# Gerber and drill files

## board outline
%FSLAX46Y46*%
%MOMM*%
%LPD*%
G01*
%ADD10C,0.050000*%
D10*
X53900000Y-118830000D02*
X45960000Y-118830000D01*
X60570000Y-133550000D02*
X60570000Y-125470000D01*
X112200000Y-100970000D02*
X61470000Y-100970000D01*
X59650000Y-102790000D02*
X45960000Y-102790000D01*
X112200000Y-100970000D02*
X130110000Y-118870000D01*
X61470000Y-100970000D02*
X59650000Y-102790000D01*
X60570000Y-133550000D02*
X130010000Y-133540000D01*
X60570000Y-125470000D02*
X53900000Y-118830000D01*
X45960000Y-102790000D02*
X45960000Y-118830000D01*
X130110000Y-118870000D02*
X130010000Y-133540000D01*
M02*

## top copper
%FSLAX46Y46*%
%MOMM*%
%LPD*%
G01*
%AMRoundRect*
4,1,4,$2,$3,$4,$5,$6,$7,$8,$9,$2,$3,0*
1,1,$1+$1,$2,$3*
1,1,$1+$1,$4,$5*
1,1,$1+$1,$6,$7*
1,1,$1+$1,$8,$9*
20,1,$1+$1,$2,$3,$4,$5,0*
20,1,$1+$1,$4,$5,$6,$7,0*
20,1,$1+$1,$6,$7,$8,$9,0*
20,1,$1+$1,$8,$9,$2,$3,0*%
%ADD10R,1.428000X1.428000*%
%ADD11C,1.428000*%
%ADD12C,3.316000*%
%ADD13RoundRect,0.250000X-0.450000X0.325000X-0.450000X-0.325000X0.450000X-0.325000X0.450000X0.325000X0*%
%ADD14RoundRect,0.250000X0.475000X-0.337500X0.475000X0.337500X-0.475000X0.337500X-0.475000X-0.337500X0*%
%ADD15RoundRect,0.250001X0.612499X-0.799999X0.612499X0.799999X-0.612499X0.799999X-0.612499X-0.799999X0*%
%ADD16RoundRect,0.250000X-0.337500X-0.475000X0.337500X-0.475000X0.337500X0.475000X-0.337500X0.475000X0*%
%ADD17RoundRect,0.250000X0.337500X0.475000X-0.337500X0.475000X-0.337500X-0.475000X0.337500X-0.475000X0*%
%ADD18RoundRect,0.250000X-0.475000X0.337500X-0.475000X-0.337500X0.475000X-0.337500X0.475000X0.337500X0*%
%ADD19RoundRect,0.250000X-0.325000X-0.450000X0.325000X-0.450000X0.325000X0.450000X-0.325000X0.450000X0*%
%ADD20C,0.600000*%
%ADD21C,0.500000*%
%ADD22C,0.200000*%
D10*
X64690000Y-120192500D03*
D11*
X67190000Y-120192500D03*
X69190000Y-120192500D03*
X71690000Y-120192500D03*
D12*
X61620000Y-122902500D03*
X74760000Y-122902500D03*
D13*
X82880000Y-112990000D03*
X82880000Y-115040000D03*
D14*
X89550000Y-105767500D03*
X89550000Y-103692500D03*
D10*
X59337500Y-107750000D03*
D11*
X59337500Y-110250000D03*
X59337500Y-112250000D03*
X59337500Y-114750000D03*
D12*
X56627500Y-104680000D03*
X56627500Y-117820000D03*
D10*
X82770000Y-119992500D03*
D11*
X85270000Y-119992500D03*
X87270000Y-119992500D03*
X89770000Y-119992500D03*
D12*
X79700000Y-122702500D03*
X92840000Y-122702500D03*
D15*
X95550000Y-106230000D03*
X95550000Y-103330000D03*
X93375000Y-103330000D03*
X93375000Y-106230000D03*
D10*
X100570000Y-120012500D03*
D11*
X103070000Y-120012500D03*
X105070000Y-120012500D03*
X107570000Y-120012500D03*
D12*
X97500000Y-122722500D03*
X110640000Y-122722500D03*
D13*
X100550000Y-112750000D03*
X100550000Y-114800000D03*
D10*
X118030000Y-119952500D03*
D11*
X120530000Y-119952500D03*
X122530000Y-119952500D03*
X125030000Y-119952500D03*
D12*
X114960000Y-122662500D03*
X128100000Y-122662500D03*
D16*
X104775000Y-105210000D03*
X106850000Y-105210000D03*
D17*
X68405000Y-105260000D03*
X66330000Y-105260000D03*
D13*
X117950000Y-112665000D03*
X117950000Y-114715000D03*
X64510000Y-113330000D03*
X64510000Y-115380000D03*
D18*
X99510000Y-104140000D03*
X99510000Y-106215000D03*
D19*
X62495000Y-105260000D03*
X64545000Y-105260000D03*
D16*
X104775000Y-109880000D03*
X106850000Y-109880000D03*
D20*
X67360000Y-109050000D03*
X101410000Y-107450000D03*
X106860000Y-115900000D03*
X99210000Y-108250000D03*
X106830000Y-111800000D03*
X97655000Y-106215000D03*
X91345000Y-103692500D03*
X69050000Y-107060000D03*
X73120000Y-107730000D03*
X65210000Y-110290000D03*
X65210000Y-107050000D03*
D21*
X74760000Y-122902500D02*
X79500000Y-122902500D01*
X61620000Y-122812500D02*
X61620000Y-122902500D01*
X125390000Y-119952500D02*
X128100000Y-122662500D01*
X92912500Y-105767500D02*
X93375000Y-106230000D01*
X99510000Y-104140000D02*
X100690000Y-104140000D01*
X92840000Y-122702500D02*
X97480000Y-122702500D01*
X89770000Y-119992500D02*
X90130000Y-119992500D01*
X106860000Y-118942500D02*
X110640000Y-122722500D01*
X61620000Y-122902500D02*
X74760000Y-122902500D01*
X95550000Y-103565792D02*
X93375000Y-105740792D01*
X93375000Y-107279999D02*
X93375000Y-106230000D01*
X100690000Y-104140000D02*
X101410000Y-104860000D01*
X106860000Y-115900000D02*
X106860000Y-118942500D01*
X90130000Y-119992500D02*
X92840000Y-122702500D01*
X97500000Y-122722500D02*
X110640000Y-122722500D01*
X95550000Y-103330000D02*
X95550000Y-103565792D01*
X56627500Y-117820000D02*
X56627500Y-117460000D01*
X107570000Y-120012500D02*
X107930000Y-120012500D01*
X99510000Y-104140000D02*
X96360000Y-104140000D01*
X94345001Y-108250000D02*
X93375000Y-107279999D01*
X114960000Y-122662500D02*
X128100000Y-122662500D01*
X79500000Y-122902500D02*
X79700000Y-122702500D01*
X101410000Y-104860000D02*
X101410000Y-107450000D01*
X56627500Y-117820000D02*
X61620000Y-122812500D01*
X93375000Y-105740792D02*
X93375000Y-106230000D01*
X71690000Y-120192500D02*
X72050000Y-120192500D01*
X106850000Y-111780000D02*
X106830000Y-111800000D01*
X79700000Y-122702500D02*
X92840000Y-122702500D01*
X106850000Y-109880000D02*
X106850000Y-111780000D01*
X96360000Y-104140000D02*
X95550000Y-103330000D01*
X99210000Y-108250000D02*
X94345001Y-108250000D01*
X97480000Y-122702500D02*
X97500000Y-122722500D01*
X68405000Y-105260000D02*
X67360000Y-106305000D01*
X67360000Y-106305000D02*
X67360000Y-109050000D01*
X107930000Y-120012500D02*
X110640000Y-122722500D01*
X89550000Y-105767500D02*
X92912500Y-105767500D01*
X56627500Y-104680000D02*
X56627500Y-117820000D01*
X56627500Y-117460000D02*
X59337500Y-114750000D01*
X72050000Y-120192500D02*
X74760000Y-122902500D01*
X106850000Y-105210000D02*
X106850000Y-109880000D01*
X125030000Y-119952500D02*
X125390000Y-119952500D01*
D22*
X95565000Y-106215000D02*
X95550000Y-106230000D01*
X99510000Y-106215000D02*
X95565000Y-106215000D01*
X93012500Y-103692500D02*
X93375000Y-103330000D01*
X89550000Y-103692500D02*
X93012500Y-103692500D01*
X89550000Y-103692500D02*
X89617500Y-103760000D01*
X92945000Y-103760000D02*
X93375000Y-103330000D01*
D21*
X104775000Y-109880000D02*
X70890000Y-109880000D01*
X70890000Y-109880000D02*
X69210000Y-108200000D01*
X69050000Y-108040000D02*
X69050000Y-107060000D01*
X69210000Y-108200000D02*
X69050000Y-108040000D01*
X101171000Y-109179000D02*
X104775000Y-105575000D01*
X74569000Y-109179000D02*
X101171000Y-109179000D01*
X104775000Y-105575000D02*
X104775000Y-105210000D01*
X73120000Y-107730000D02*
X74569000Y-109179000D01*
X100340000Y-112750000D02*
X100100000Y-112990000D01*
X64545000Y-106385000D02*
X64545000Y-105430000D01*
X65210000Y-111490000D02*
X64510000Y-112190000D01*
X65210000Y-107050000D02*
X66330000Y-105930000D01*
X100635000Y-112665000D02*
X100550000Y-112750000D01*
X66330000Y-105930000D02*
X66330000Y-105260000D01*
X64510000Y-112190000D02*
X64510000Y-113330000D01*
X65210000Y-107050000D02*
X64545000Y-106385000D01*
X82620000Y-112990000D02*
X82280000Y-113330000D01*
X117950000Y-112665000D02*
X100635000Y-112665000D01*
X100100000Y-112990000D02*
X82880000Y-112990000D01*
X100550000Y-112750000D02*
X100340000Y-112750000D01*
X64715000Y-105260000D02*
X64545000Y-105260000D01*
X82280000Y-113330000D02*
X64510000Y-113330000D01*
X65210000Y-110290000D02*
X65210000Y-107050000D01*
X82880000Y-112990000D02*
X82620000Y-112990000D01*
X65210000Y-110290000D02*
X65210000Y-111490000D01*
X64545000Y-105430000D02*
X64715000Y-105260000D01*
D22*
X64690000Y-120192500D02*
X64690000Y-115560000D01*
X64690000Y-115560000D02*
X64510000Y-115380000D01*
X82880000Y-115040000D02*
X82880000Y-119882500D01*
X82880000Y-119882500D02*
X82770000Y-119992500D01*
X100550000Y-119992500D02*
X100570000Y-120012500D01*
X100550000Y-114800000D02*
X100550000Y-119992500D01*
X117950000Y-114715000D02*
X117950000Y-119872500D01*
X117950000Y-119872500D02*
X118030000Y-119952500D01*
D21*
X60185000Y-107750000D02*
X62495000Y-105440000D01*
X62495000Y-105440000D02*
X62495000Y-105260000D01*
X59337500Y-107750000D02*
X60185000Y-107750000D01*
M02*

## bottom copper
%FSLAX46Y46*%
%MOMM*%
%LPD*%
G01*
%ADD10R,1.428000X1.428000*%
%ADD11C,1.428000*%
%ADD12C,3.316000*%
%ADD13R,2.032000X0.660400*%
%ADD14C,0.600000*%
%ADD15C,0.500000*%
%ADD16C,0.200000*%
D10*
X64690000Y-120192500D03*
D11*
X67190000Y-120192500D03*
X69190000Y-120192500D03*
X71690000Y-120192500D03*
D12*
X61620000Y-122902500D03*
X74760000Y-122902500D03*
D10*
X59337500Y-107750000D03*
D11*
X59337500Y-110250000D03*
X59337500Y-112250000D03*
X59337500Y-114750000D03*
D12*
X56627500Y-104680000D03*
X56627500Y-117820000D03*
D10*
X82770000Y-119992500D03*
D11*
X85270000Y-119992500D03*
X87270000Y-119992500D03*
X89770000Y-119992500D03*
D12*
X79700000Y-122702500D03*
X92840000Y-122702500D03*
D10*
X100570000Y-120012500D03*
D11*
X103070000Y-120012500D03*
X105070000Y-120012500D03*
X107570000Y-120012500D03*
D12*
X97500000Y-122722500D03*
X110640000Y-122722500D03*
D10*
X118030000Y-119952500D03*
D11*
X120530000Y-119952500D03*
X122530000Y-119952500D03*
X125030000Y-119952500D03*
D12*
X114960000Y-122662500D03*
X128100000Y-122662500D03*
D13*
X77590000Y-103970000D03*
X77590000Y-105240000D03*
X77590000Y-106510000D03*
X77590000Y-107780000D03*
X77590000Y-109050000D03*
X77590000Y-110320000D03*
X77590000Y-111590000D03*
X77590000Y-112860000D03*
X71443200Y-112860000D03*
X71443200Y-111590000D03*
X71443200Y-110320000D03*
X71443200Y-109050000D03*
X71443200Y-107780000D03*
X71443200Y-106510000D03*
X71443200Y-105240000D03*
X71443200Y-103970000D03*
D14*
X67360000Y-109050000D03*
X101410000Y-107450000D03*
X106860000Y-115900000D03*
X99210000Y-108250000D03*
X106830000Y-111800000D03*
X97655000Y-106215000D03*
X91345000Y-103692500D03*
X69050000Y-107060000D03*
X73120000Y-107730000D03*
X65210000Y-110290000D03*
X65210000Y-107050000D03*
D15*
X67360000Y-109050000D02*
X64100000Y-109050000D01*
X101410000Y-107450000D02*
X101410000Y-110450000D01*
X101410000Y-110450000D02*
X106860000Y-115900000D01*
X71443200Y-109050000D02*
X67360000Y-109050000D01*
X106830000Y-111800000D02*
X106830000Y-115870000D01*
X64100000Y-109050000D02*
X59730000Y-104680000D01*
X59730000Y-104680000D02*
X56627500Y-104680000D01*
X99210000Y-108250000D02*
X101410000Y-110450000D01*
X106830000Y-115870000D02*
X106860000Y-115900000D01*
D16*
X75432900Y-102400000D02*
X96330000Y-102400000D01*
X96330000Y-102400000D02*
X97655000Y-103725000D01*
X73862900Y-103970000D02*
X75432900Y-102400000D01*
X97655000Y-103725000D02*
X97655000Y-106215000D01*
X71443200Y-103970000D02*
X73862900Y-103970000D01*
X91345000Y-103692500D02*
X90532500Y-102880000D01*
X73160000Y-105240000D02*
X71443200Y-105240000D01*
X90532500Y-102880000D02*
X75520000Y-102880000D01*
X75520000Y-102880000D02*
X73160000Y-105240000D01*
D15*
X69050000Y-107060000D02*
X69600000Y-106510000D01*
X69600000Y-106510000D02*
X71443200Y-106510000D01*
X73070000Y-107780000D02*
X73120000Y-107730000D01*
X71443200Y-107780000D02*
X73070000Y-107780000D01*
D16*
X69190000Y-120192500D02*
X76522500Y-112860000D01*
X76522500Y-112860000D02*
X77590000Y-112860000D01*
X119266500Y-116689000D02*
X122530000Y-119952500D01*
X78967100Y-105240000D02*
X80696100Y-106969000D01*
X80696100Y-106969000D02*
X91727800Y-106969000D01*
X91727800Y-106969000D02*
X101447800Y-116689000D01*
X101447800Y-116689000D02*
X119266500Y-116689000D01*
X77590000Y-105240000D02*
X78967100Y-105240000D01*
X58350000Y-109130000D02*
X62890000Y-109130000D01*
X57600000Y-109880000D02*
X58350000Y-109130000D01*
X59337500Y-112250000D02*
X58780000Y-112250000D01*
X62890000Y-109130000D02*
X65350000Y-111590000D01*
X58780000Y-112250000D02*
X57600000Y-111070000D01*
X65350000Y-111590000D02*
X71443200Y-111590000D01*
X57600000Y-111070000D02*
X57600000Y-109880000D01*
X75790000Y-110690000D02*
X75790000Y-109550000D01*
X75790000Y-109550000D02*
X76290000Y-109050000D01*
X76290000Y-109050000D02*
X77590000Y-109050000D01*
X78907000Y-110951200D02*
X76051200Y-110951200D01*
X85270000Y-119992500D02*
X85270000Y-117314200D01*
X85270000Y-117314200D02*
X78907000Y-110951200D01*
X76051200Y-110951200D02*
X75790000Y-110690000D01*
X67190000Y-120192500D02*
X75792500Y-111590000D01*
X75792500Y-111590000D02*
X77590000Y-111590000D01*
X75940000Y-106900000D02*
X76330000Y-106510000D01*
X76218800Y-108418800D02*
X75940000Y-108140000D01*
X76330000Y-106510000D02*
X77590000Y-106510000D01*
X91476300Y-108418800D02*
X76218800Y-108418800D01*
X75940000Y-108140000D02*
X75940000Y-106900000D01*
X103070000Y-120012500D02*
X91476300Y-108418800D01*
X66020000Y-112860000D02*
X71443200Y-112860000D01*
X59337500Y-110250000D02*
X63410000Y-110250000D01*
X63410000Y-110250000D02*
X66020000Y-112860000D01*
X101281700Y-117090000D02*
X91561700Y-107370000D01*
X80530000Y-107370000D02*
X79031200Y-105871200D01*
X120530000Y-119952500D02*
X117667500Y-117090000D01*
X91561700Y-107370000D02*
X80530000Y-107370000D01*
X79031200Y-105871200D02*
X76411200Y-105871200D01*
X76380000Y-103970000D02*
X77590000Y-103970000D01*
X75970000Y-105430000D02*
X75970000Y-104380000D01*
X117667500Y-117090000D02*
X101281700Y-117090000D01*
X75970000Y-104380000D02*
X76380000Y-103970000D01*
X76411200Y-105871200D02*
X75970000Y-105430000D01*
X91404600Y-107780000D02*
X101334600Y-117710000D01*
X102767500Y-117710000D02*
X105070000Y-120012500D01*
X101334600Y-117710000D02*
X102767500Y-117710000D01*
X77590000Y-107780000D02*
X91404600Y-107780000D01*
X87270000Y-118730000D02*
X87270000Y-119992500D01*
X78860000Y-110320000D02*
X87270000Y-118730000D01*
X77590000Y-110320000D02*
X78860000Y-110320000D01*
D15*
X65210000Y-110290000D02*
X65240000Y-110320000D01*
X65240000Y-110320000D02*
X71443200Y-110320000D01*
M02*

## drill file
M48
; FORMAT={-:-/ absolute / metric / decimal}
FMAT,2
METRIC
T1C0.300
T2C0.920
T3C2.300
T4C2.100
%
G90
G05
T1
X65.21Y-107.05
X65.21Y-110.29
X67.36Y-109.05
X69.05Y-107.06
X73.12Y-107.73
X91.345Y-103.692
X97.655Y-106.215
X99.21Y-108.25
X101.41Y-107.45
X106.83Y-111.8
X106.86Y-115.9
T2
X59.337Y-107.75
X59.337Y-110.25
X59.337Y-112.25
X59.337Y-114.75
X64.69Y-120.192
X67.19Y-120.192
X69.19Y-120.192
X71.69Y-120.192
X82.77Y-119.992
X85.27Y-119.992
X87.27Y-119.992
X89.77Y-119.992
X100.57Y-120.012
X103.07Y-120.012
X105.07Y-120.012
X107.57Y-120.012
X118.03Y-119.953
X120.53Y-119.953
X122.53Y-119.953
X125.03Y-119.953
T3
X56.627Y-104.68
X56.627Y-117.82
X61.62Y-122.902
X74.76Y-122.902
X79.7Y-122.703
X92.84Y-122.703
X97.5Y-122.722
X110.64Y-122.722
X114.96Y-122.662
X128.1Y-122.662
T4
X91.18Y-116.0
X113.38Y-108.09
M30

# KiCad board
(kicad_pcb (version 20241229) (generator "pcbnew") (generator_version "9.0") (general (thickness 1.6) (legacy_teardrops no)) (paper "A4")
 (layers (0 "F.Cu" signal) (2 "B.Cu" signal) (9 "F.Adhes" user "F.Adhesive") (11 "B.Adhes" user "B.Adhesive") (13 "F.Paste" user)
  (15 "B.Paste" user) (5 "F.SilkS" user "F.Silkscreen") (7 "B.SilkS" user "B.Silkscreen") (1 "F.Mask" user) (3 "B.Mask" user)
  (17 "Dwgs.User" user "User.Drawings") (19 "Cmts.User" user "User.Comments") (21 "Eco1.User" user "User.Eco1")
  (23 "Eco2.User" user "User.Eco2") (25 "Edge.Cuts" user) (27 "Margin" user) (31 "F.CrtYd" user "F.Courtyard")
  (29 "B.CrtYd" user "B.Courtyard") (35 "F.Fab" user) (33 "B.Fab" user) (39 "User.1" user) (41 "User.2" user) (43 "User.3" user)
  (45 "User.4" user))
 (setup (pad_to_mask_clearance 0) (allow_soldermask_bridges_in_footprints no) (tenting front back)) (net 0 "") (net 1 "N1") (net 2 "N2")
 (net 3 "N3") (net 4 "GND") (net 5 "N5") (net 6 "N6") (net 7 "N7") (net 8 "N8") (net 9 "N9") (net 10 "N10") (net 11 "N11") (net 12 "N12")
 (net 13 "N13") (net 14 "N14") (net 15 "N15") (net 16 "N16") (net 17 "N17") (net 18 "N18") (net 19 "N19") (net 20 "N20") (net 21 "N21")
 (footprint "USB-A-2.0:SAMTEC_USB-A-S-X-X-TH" (layer "F.Cu") (at 68.19 122.9025)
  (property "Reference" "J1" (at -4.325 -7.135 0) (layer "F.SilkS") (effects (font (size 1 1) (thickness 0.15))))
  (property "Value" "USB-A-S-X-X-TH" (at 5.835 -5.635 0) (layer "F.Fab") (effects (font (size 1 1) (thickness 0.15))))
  (pad "01" thru_hole rect (at -3.5 -2.71) (size 1.428 1.428) (drill 0.92) (layers "*.Cu" "*.Mask") (remove_unused_layers no) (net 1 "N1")
   (solder_mask_margin 0.102))
  (pad "02" thru_hole circle (at -1 -2.71) (size 1.428 1.428) (drill 0.92) (layers "*.Cu" "*.Mask") (remove_unused_layers no) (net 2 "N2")
   (solder_mask_margin 0.102))
  (pad "03" thru_hole circle (at 1 -2.71) (size 1.428 1.428) (drill 0.92) (layers "*.Cu" "*.Mask") (remove_unused_layers no) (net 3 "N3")
   (solder_mask_margin 0.102))
  (pad "04" thru_hole circle (at 3.5 -2.71) (size 1.428 1.428) (drill 0.92) (layers "*.Cu" "*.Mask") (remove_unused_layers no) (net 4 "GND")
   (solder_mask_margin 0.102))
  (pad "S1" thru_hole circle (at -6.57 0) (size 3.316 3.316) (drill 2.3) (layers "*.Cu" "*.Mask") (remove_unused_layers no) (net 4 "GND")
   (solder_mask_margin 0.102))
  (pad "S2" thru_hole circle (at 6.57 0) (size 3.316 3.316) (drill 2.3) (layers "*.Cu" "*.Mask") (remove_unused_layers no) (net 4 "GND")
   (solder_mask_margin 0.102)))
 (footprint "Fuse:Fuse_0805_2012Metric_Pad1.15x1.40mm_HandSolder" (layer "F.Cu") (at 82.88 114.015 -90)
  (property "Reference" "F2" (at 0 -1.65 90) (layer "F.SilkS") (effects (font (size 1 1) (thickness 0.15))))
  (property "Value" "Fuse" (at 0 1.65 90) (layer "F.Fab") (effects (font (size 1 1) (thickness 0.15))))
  (pad "1" smd roundrect (at -1.025 0 270) (size 1.15 1.4) (layers "F.Cu" "F.Mask" "F.Paste") (roundrect_rratio 0.217391) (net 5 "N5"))
  (pad "2" smd roundrect (at 1.025 0 270) (size 1.15 1.4) (layers "F.Cu" "F.Mask" "F.Paste") (roundrect_rratio 0.217391) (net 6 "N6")))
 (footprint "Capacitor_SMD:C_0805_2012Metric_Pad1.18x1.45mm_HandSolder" (layer "F.Cu") (at 89.55 104.73 90)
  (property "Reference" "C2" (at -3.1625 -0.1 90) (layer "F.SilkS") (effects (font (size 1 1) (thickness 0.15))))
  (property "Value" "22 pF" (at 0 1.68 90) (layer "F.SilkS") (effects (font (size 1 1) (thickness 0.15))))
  (pad "1" smd roundrect (at -1.0375 0 90) (size 1.175 1.45) (layers "F.Cu" "F.Mask" "F.Paste") (roundrect_rratio 0.212766) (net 4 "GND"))
  (pad "2" smd roundrect (at 1.0375 0 90) (size 1.175 1.45) (layers "F.Cu" "F.Mask" "F.Paste") (roundrect_rratio 0.212766) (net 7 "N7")))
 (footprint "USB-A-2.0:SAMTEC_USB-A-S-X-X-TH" (layer "F.Cu") (at 56.6275 111.25 -90)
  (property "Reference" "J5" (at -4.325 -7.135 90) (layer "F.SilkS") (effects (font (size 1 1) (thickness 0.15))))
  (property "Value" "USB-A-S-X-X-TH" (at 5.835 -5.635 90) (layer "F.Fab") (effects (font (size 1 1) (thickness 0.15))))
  (pad "01" thru_hole rect (at -3.5 -2.71 270) (size 1.428 1.428) (drill 0.92) (layers "*.Cu" "*.Mask") (remove_unused_layers no)
   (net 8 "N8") (solder_mask_margin 0.102))
  (pad "02" thru_hole circle (at -1 -2.71 270) (size 1.428 1.428) (drill 0.92) (layers "*.Cu" "*.Mask") (remove_unused_layers no)
   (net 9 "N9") (solder_mask_margin 0.102))
  (pad "03" thru_hole circle (at 1 -2.71 270) (size 1.428 1.428) (drill 0.92) (layers "*.Cu" "*.Mask") (remove_unused_layers no)
   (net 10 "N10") (solder_mask_margin 0.102))
  (pad "04" thru_hole circle (at 3.5 -2.71 270) (size 1.428 1.428) (drill 0.92) (layers "*.Cu" "*.Mask") (remove_unused_layers no)
   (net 4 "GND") (solder_mask_margin 0.102))
  (pad "S1" thru_hole circle (at -6.57 0 270) (size 3.316 3.316) (drill 2.3) (layers "*.Cu" "*.Mask") (remove_unused_layers no)
   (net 4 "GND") (solder_mask_margin 0.102))
  (pad "S2" thru_hole circle (at 6.57 0 270) (size 3.316 3.316) (drill 2.3) (layers "*.Cu" "*.Mask") (remove_unused_layers no) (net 4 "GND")
   (solder_mask_margin 0.102)))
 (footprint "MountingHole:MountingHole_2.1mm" (layer "F.Cu") (at 91.18 116)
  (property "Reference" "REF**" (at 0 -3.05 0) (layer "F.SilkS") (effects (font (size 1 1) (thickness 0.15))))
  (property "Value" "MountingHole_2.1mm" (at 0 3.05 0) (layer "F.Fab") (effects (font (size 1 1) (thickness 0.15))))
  (pad "" np_thru_hole circle (at 0 0) (size 2.1 2.1) (drill 2.1) (layers "*.Cu" "*.Mask")))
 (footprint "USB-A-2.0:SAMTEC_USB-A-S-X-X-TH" (layer "F.Cu") (at 86.27 122.7025)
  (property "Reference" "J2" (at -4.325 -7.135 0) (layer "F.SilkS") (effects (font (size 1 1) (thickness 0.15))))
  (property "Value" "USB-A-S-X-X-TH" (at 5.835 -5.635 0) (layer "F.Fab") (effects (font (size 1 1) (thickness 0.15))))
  (pad "01" thru_hole rect (at -3.5 -2.71) (size 1.428 1.428) (drill 0.92) (layers "*.Cu" "*.Mask") (remove_unused_layers no) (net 6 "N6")
   (solder_mask_margin 0.102))
  (pad "02" thru_hole circle (at -1 -2.71) (size 1.428 1.428) (drill 0.92) (layers "*.Cu" "*.Mask") (remove_unused_layers no) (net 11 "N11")
   (solder_mask_margin 0.102))
  (pad "03" thru_hole circle (at 1 -2.71) (size 1.428 1.428) (drill 0.92) (layers "*.Cu" "*.Mask") (remove_unused_layers no) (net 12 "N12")
   (solder_mask_margin 0.102))
  (pad "04" thru_hole circle (at 3.5 -2.71) (size 1.428 1.428) (drill 0.92) (layers "*.Cu" "*.Mask") (remove_unused_layers no) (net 4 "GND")
   (solder_mask_margin 0.102))
  (pad "S1" thru_hole circle (at -6.57 0) (size 3.316 3.316) (drill 2.3) (layers "*.Cu" "*.Mask") (remove_unused_layers no) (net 4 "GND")
   (solder_mask_margin 0.102))
  (pad "S2" thru_hole circle (at 6.57 0) (size 3.316 3.316) (drill 2.3) (layers "*.Cu" "*.Mask") (remove_unused_layers no) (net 4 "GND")
   (solder_mask_margin 0.102)))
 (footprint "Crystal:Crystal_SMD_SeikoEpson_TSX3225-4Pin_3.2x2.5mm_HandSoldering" (layer "F.Cu") (at 94.4625 104.78 90)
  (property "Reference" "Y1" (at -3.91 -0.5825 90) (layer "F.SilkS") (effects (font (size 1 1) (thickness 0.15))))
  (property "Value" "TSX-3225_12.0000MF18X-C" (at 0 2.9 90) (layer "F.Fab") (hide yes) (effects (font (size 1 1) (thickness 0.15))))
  (pad "1" smd roundrect (at -1.45 1.0875 90) (size 2.1 1.725) (layers "F.Cu" "F.Mask" "F.Paste") (roundrect_rratio 0.144928) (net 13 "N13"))
  (pad "2" smd roundrect (at 1.45 1.0875 90) (size 2.1 1.725) (layers "F.Cu" "F.Mask" "F.Paste") (roundrect_rratio 0.144928) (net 4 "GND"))
  (pad "3" smd roundrect (at 1.45 -1.0875 90) (size 2.1 1.725) (layers "F.Cu" "F.Mask" "F.Paste") (roundrect_rratio 0.144928) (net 7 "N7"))
  (pad "4" smd roundrect (at -1.45 -1.0875 90) (size 2.1 1.725) (layers "F.Cu" "F.Mask" "F.Paste") (roundrect_rratio 0.144928) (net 4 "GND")))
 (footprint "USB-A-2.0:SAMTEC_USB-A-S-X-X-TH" (layer "F.Cu") (at 104.07 122.7225)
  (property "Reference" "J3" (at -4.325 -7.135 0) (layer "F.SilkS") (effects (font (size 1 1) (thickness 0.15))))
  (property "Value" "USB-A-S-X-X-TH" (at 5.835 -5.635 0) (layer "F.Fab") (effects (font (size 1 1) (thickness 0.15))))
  (pad "01" thru_hole rect (at -3.5 -2.71) (size 1.428 1.428) (drill 0.92) (layers "*.Cu" "*.Mask") (remove_unused_layers no) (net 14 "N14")
   (solder_mask_margin 0.102))
  (pad "02" thru_hole circle (at -1 -2.71) (size 1.428 1.428) (drill 0.92) (layers "*.Cu" "*.Mask") (remove_unused_layers no) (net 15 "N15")
   (solder_mask_margin 0.102))
  (pad "03" thru_hole circle (at 1 -2.71) (size 1.428 1.428) (drill 0.92) (layers "*.Cu" "*.Mask") (remove_unused_layers no) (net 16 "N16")
   (solder_mask_margin 0.102))
  (pad "04" thru_hole circle (at 3.5 -2.71) (size 1.428 1.428) (drill 0.92) (layers "*.Cu" "*.Mask") (remove_unused_layers no) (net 4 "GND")
   (solder_mask_margin 0.102))
  (pad "S1" thru_hole circle (at -6.57 0) (size 3.316 3.316) (drill 2.3) (layers "*.Cu" "*.Mask") (remove_unused_layers no) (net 4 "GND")
   (solder_mask_margin 0.102))
  (pad "S2" thru_hole circle (at 6.57 0) (size 3.316 3.316) (drill 2.3) (layers "*.Cu" "*.Mask") (remove_unused_layers no) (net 4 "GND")
   (solder_mask_margin 0.102)))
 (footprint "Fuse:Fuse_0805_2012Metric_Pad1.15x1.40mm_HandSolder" (layer "F.Cu") (at 100.55 113.775 -90)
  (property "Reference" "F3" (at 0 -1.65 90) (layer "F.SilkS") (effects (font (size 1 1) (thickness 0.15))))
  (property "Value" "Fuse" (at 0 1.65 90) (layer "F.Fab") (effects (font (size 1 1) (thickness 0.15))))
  (pad "1" smd roundrect (at -1.025 0 270) (size 1.15 1.4) (layers "F.Cu" "F.Mask" "F.Paste") (roundrect_rratio 0.217391) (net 5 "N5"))
  (pad "2" smd roundrect (at 1.025 0 270) (size 1.15 1.4) (layers "F.Cu" "F.Mask" "F.Paste") (roundrect_rratio 0.217391) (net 14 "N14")))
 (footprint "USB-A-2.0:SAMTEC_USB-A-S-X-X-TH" (layer "F.Cu") (at 121.53 122.6625)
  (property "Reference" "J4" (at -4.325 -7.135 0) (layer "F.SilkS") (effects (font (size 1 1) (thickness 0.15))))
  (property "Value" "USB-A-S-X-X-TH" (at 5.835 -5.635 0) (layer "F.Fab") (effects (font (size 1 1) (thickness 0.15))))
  (pad "01" thru_hole rect (at -3.5 -2.71) (size 1.428 1.428) (drill 0.92) (layers "*.Cu" "*.Mask") (remove_unused_layers no) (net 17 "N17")
   (solder_mask_margin 0.102))
  (pad "02" thru_hole circle (at -1 -2.71) (size 1.428 1.428) (drill 0.92) (layers "*.Cu" "*.Mask") (remove_unused_layers no) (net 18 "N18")
   (solder_mask_margin 0.102))
  (pad "03" thru_hole circle (at 1 -2.71) (size 1.428 1.428) (drill 0.92) (layers "*.Cu" "*.Mask") (remove_unused_layers no) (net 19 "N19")
   (solder_mask_margin 0.102))
  (pad "04" thru_hole circle (at 3.5 -2.71) (size 1.428 1.428) (drill 0.92) (layers "*.Cu" "*.Mask") (remove_unused_layers no) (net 4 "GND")
   (solder_mask_margin 0.102))
  (pad "S1" thru_hole circle (at -6.57 0) (size 3.316 3.316) (drill 2.3) (layers "*.Cu" "*.Mask") (remove_unused_layers no) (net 4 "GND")
   (solder_mask_margin 0.102))
  (pad "S2" thru_hole circle (at 6.57 0) (size 3.316 3.316) (drill 2.3) (layers "*.Cu" "*.Mask") (remove_unused_layers no) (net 4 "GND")
   (solder_mask_margin 0.102)))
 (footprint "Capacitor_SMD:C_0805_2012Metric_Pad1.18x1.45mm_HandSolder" (layer "F.Cu") (at 105.8125 105.21)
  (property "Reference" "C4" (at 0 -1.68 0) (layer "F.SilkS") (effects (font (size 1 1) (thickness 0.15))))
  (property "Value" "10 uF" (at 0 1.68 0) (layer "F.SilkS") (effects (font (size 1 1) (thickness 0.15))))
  (pad "1" smd roundrect (at -1.0375 0) (size 1.175 1.45) (layers "F.Cu" "F.Mask" "F.Paste") (roundrect_rratio 0.212766) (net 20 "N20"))
  (pad "2" smd roundrect (at 1.0375 0) (size 1.175 1.45) (layers "F.Cu" "F.Mask" "F.Paste") (roundrect_rratio 0.212766) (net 4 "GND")))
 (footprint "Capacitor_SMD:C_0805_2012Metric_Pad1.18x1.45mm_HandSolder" (layer "F.Cu") (at 67.3675 105.26 180)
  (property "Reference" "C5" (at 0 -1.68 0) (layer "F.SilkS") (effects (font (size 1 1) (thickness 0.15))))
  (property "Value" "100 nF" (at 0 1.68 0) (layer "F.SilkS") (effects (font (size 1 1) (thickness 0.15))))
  (pad "1" smd roundrect (at -1.0375 0 180) (size 1.175 1.45) (layers "F.Cu" "F.Mask" "F.Paste") (roundrect_rratio 0.212766) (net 4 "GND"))
  (pad "2" smd roundrect (at 1.0375 0 180) (size 1.175 1.45) (layers "F.Cu" "F.Mask" "F.Paste") (roundrect_rratio 0.212766) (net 5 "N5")))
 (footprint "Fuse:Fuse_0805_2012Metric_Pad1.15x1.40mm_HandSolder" (layer "F.Cu") (at 117.95 113.69 -90)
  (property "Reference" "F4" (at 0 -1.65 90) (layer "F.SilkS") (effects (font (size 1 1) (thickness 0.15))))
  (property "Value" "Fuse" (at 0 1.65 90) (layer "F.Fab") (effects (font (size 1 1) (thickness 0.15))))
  (pad "1" smd roundrect (at -1.025 0 270) (size 1.15 1.4) (layers "F.Cu" "F.Mask" "F.Paste") (roundrect_rratio 0.217391) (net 5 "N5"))
  (pad "2" smd roundrect (at 1.025 0 270) (size 1.15 1.4) (layers "F.Cu" "F.Mask" "F.Paste") (roundrect_rratio 0.217391) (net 17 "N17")))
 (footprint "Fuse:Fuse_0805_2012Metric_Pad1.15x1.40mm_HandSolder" (layer "F.Cu") (at 64.51 114.355 -90)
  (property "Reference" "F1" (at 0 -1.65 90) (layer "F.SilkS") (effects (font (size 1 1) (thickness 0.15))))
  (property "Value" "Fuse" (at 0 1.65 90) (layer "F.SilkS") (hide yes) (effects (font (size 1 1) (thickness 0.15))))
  (pad "1" smd roundrect (at -1.025 0 270) (size 1.15 1.4) (layers "F.Cu" "F.Mask" "F.Paste") (roundrect_rratio 0.217391) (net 5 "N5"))
  (pad "2" smd roundrect (at 1.025 0 270) (size 1.15 1.4) (layers "F.Cu" "F.Mask" "F.Paste") (roundrect_rratio 0.217391) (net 1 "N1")))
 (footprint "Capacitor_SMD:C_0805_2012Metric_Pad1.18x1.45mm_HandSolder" (layer "F.Cu") (at 99.51 105.1775 -90)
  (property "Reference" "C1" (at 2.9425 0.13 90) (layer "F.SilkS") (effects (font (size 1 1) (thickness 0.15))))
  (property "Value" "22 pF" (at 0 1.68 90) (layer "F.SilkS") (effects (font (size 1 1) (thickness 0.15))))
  (pad "1" smd roundrect (at -1.0375 0 270) (size 1.175 1.45) (layers "F.Cu" "F.Mask" "F.Paste") (roundrect_rratio 0.212766) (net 4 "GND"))
  (pad "2" smd roundrect (at 1.0375 0 270) (size 1.175 1.45) (layers "F.Cu" "F.Mask" "F.Paste") (roundrect_rratio 0.212766) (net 13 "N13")))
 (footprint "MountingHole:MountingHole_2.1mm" (layer "F.Cu") (at 113.38 108.09)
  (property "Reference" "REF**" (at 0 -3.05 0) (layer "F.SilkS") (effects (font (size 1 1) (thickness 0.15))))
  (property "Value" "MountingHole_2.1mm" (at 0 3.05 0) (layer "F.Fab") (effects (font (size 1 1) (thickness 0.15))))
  (pad "" np_thru_hole circle (at 0 0) (size 2.1 2.1) (drill 2.1) (layers "*.Cu" "*.Mask")))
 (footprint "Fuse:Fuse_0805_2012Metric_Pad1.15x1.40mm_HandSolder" (layer "F.Cu") (at 63.52 105.26)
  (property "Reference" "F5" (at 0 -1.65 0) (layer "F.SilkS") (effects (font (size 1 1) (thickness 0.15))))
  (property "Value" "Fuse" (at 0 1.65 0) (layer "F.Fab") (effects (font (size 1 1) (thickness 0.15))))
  (pad "1" smd roundrect (at -1.025 0) (size 1.15 1.4) (layers "F.Cu" "F.Mask" "F.Paste") (roundrect_rratio 0.217391) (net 8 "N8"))
  (pad "2" smd roundrect (at 1.025 0) (size 1.15 1.4) (layers "F.Cu" "F.Mask" "F.Paste") (roundrect_rratio 0.217391) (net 5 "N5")))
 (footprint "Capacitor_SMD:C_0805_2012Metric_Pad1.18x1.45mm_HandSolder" (layer "F.Cu") (at 105.8125 109.88)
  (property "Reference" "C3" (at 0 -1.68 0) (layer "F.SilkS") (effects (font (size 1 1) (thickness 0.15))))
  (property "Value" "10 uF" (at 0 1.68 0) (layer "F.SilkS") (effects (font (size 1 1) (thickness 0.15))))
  (pad "1" smd roundrect (at -1.0375 0) (size 1.175 1.45) (layers "F.Cu" "F.Mask" "F.Paste") (roundrect_rratio 0.212766) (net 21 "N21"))
  (pad "2" smd roundrect (at 1.0375 0) (size 1.175 1.45) (layers "F.Cu" "F.Mask" "F.Paste") (roundrect_rratio 0.212766) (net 4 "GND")))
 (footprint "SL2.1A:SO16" (layer "B.Cu") (at 74.5166 108.415 -90)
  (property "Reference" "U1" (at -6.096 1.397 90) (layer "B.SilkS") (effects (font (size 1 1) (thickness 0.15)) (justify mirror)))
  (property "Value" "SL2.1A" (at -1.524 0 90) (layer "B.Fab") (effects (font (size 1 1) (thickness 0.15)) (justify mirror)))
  (pad "1" smd rect (at -4.445 -3.0734 270) (size 0.6604 2.032) (layers "B.Cu" "B.Mask" "B.Paste") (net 18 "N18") (solder_mask_margin 0.102))
  (pad "2" smd rect (at -3.175 -3.0734 270) (size 0.6604 2.032) (layers "B.Cu" "B.Mask" "B.Paste") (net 19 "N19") (solder_mask_margin 0.102))
  (pad "3" smd rect (at -1.905 -3.0734 270) (size 0.6604 2.032) (layers "B.Cu" "B.Mask" "B.Paste") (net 15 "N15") (solder_mask_margin 0.102))
  (pad "4" smd rect (at -0.635 -3.0734 270) (size 0.6604 2.032) (layers "B.Cu" "B.Mask" "B.Paste") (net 16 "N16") (solder_mask_margin 0.102))
  (pad "5" smd rect (at 0.635 -3.0734 270) (size 0.6604 2.032) (layers "B.Cu" "B.Mask" "B.Paste") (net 11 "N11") (solder_mask_margin 0.102))
  (pad "6" smd rect (at 1.905 -3.0734 270) (size 0.6604 2.032) (layers "B.Cu" "B.Mask" "B.Paste") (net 12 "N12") (solder_mask_margin 0.102))
  (pad "7" smd rect (at 3.175 -3.0734 270) (size 0.6604 2.032) (layers "B.Cu" "B.Mask" "B.Paste") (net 2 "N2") (solder_mask_margin 0.102))
  (pad "8" smd rect (at 4.445 -3.0734 270) (size 0.6604 2.032) (layers "B.Cu" "B.Mask" "B.Paste") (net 3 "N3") (solder_mask_margin 0.102))
  (pad "9" smd rect (at 4.445 3.0734 270) (size 0.6604 2.032) (layers "B.Cu" "B.Mask" "B.Paste") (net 9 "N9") (solder_mask_margin 0.102))
  (pad "10" smd rect (at 3.175 3.0734 270) (size 0.6604 2.032) (layers "B.Cu" "B.Mask" "B.Paste") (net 10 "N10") (solder_mask_margin 0.102))
  (pad "11" smd rect (at 1.905 3.0734 270) (size 0.6604 2.032) (layers "B.Cu" "B.Mask" "B.Paste") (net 5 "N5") (solder_mask_margin 0.102))
  (pad "12" smd rect (at 0.635 3.0734 270) (size 0.6604 2.032) (layers "B.Cu" "B.Mask" "B.Paste") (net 4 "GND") (solder_mask_margin 0.102))
  (pad "13" smd rect (at -0.635 3.0734 270) (size 0.6604 2.032) (layers "B.Cu" "B.Mask" "B.Paste") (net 20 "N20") (solder_mask_margin 0.102))
  (pad "14" smd rect (at -1.905 3.0734 270) (size 0.6604 2.032) (layers "B.Cu" "B.Mask" "B.Paste") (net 21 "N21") (solder_mask_margin 0.102))
  (pad "15" smd rect (at -3.175 3.0734 270) (size 0.6604 2.032) (layers "B.Cu" "B.Mask" "B.Paste") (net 7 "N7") (solder_mask_margin 0.102))
  (pad "16" smd rect (at -4.445 3.0734 270) (size 0.6604 2.032) (layers "B.Cu" "B.Mask" "B.Paste") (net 13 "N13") (solder_mask_margin 0.102)))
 (gr_line (start 53.9 118.83) (end 45.96 118.83) (stroke (width 0.05) (type default)) (layer "Edge.Cuts"))
 (gr_line (start 60.57 133.55) (end 60.57 125.47) (stroke (width 0.05) (type default)) (layer "Edge.Cuts"))
 (gr_line (start 112.2 100.97) (end 61.47 100.97) (stroke (width 0.05) (type default)) (layer "Edge.Cuts"))
 (gr_line (start 59.65 102.79) (end 45.96 102.79) (stroke (width 0.05) (type default)) (layer "Edge.Cuts"))
 (gr_line (start 112.2 100.97) (end 130.11 118.87) (stroke (width 0.05) (type default)) (layer "Edge.Cuts"))
 (gr_line (start 61.47 100.97) (end 59.65 102.79) (stroke (width 0.05) (type default)) (layer "Edge.Cuts"))
 (gr_line (start 60.57 133.55) (end 130.01 133.54) (stroke (width 0.05) (type default)) (layer "Edge.Cuts"))
 (gr_line (start 60.57 125.47) (end 53.9 118.83) (stroke (width 0.05) (type default)) (layer "Edge.Cuts"))
 (gr_line (start 45.96 102.79) (end 45.96 118.83) (stroke (width 0.05) (type default)) (layer "Edge.Cuts"))
 (gr_line (start 130.11 118.87) (end 130.01 133.54) (stroke (width 0.05) (type default)) (layer "Edge.Cuts"))
 (segment (start 74.76 122.9025) (end 79.5 122.9025) (width 0.5) (layer "F.Cu") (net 4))
 (segment (start 61.62 122.8125) (end 61.62 122.9025) (width 0.5) (layer "F.Cu") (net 4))
 (segment (start 125.39 119.9525) (end 128.1 122.6625) (width 0.5) (layer "F.Cu") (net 4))
 (segment (start 92.9125 105.7675) (end 93.375 106.23) (width 0.5) (layer "F.Cu") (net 4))
 (segment (start 99.51 104.14) (end 100.69 104.14) (width 0.5) (layer "F.Cu") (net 4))
 (segment (start 92.84 122.7025) (end 97.48 122.7025) (width 0.5) (layer "F.Cu") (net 4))
 (segment (start 89.77 119.9925) (end 90.13 119.9925) (width 0.5) (layer "F.Cu") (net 4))
 (segment (start 106.86 118.9425) (end 110.64 122.7225) (width 0.5) (layer "F.Cu") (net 4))
 (segment (start 61.62 122.9025) (end 74.76 122.9025) (width 0.5) (layer "F.Cu") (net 4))
 (segment (start 95.55 103.565792) (end 93.375 105.740792) (width 0.5) (layer "F.Cu") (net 4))
 (segment (start 93.375 107.279999) (end 93.375 106.23) (width 0.5) (layer "F.Cu") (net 4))
 (segment (start 100.69 104.14) (end 101.41 104.86) (width 0.5) (layer "F.Cu") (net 4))
 (segment (start 106.86 115.9) (end 106.86 118.9425) (width 0.5) (layer "F.Cu") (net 4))
 (segment (start 90.13 119.9925) (end 92.84 122.7025) (width 0.5) (layer "F.Cu") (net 4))
 (segment (start 97.5 122.7225) (end 110.64 122.7225) (width 0.5) (layer "F.Cu") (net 4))
 (segment (start 95.55 103.33) (end 95.55 103.565792) (width 0.5) (layer "F.Cu") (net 4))
 (segment (start 56.6275 117.82) (end 56.6275 117.46) (width 0.5) (layer "F.Cu") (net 4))
 (segment (start 107.57 120.0125) (end 107.93 120.0125) (width 0.5) (layer "F.Cu") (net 4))
 (segment (start 99.51 104.14) (end 96.36 104.14) (width 0.5) (layer "F.Cu") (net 4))
 (segment (start 94.345001 108.25) (end 93.375 107.279999) (width 0.5) (layer "F.Cu") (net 4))
 (segment (start 114.96 122.6625) (end 128.1 122.6625) (width 0.5) (layer "F.Cu") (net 4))
 (segment (start 79.5 122.9025) (end 79.7 122.7025) (width 0.5) (layer "F.Cu") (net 4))
 (segment (start 101.41 104.86) (end 101.41 107.45) (width 0.5) (layer "F.Cu") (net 4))
 (segment (start 56.6275 117.82) (end 61.62 122.8125) (width 0.5) (layer "F.Cu") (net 4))
 (segment (start 93.375 105.740792) (end 93.375 106.23) (width 0.5) (layer "F.Cu") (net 4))
 (segment (start 71.69 120.1925) (end 72.05 120.1925) (width 0.5) (layer "F.Cu") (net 4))
 (segment (start 106.85 111.78) (end 106.83 111.8) (width 0.5) (layer "F.Cu") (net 4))
 (segment (start 79.7 122.7025) (end 92.84 122.7025) (width 0.5) (layer "F.Cu") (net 4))
 (segment (start 106.85 109.88) (end 106.85 111.78) (width 0.5) (layer "F.Cu") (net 4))
 (segment (start 96.36 104.14) (end 95.55 103.33) (width 0.5) (layer "F.Cu") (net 4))
 (segment (start 99.21 108.25) (end 94.345001 108.25) (width 0.5) (layer "F.Cu") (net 4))
 (segment (start 97.48 122.7025) (end 97.5 122.7225) (width 0.5) (layer "F.Cu") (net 4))
 (segment (start 68.405 105.26) (end 67.36 106.305) (width 0.5) (layer "F.Cu") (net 4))
 (segment (start 67.36 106.305) (end 67.36 109.05) (width 0.5) (layer "F.Cu") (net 4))
 (segment (start 107.93 120.0125) (end 110.64 122.7225) (width 0.5) (layer "F.Cu") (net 4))
 (segment (start 89.55 105.7675) (end 92.9125 105.7675) (width 0.5) (layer "F.Cu") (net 4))
 (segment (start 56.6275 104.68) (end 56.6275 117.82) (width 0.5) (layer "F.Cu") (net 4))
 (segment (start 56.6275 117.46) (end 59.3375 114.75) (width 0.5) (layer "F.Cu") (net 4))
 (segment (start 72.05 120.1925) (end 74.76 122.9025) (width 0.5) (layer "F.Cu") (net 4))
 (segment (start 106.85 105.21) (end 106.85 109.88) (width 0.5) (layer "F.Cu") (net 4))
 (segment (start 125.03 119.9525) (end 125.39 119.9525) (width 0.5) (layer "F.Cu") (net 4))
 (via (at 67.36 109.05) (size 0.6) (drill 0.3) (layers "F.Cu" "B.Cu") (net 4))
 (via (at 101.41 107.45) (size 0.6) (drill 0.3) (layers "F.Cu" "B.Cu") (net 4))
 (via (at 106.86 115.9) (size 0.6) (drill 0.3) (layers "F.Cu" "B.Cu") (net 4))
 (via (at 99.21 108.25) (size 0.6) (drill 0.3) (layers "F.Cu" "B.Cu") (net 4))
 (via (at 106.83 111.8) (size 0.6) (drill 0.3) (layers "F.Cu" "B.Cu") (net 4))
 (segment (start 67.36 109.05) (end 64.1 109.05) (width 0.5) (layer "B.Cu") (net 4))
 (segment (start 101.41 107.45) (end 101.41 110.45) (width 0.5) (layer "B.Cu") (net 4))
 (segment (start 101.41 110.45) (end 106.86 115.9) (width 0.5) (layer "B.Cu") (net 4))
 (segment (start 71.4432 109.05) (end 67.36 109.05) (width 0.5) (layer "B.Cu") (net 4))
 (segment (start 106.83 111.8) (end 106.83 115.87) (width 0.5) (layer "B.Cu") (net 4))
 (segment (start 64.1 109.05) (end 59.73 104.68) (width 0.5) (layer "B.Cu") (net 4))
 (segment (start 59.73 104.68) (end 56.6275 104.68) (width 0.5) (layer "B.Cu") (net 4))
 (segment (start 99.21 108.25) (end 101.41 110.45) (width 0.5) (layer "B.Cu") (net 4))
 (segment (start 106.83 115.87) (end 106.86 115.9) (width 0.5) (layer "B.Cu") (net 4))
 (segment (start 95.565 106.215) (end 95.55 106.23) (width 0.2) (layer "F.Cu") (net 13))
 (segment (start 99.51 106.215) (end 95.565 106.215) (width 0.2) (layer "F.Cu") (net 13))
 (via (at 97.655 106.215) (size 0.6) (drill 0.3) (layers "F.Cu" "B.Cu") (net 13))
 (segment (start 75.4329 102.4) (end 96.33 102.4) (width 0.2) (layer "B.Cu") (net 13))
 (segment (start 96.33 102.4) (end 97.655 103.725) (width 0.2) (layer "B.Cu") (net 13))
 (segment (start 73.8629 103.97) (end 75.4329 102.4) (width 0.2) (layer "B.Cu") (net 13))
 (segment (start 97.655 103.725) (end 97.655 106.215) (width 0.2) (layer "B.Cu") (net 13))
 (segment (start 71.4432 103.97) (end 73.8629 103.97) (width 0.2) (layer "B.Cu") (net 13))
 (segment (start 93.0125 103.6925) (end 93.375 103.33) (width 0.2) (layer "F.Cu") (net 7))
 (segment (start 89.55 103.6925) (end 93.0125 103.6925) (width 0.2) (layer "F.Cu") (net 7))
 (segment (start 89.55 103.6925) (end 89.6175 103.76) (width 0.2) (layer "F.Cu") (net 7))
 (segment (start 92.945 103.76) (end 93.375 103.33) (width 0.2) (layer "F.Cu") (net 7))
 (via (at 91.345 103.6925) (size 0.6) (drill 0.3) (layers "F.Cu" "B.Cu") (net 7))
 (segment (start 91.345 103.6925) (end 90.5325 102.88) (width 0.2) (layer "B.Cu") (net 7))
 (segment (start 73.16 105.24) (end 71.4432 105.24) (width 0.2) (layer "B.Cu") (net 7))
 (segment (start 90.5325 102.88) (end 75.52 102.88) (width 0.2) (layer "B.Cu") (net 7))
 (segment (start 75.52 102.88) (end 73.16 105.24) (width 0.2) (layer "B.Cu") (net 7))
 (segment (start 104.775 109.88) (end 70.89 109.88) (width 0.5) (layer "F.Cu") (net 21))
 (segment (start 70.89 109.88) (end 69.21 108.2) (width 0.5) (layer "F.Cu") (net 21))
 (segment (start 69.05 108.04) (end 69.05 107.06) (width 0.5) (layer "F.Cu") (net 21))
 (segment (start 69.21 108.2) (end 69.05 108.04) (width 0.5) (layer "F.Cu") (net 21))
 (via (at 69.05 107.06) (size 0.6) (drill 0.3) (layers "F.Cu" "B.Cu") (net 21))
 (segment (start 69.05 107.06) (end 69.6 106.51) (width 0.5) (layer "B.Cu") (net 21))
 (segment (start 69.6 106.51) (end 71.4432 106.51) (width 0.5) (layer "B.Cu") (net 21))
 (segment (start 101.171 109.179) (end 104.775 105.575) (width 0.5) (layer "F.Cu") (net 20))
 (segment (start 74.569 109.179) (end 101.171 109.179) (width 0.5) (layer "F.Cu") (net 20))
 (segment (start 104.775 105.575) (end 104.775 105.21) (width 0.5) (layer "F.Cu") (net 20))
 (segment (start 73.12 107.73) (end 74.569 109.179) (width 0.5) (layer "F.Cu") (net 20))
 (via (at 73.12 107.73) (size 0.6) (drill 0.3) (layers "F.Cu" "B.Cu") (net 20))
 (segment (start 73.07 107.78) (end 73.12 107.73) (width 0.5) (layer "B.Cu") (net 20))
 (segment (start 71.4432 107.78) (end 73.07 107.78) (width 0.5) (layer "B.Cu") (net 20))
 (segment (start 69.19 120.1925) (end 76.5225 112.86) (width 0.2) (layer "B.Cu") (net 3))
 (segment (start 76.5225 112.86) (end 77.59 112.86) (width 0.2) (layer "B.Cu") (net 3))
 (segment (start 119.2665 116.689) (end 122.53 119.9525) (width 0.2) (layer "B.Cu") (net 19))
 (segment (start 78.9671 105.24) (end 80.6961 106.969) (width 0.2) (layer "B.Cu") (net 19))
 (segment (start 80.6961 106.969) (end 91.7278 106.969) (width 0.2) (layer "B.Cu") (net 19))
 (segment (start 91.7278 106.969) (end 101.4478 116.689) (width 0.2) (layer "B.Cu") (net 19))
 (segment (start 101.4478 116.689) (end 119.2665 116.689) (width 0.2) (layer "B.Cu") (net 19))
 (segment (start 77.59 105.24) (end 78.9671 105.24) (width 0.2) (layer "B.Cu") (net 19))
 (segment (start 58.35 109.13) (end 62.89 109.13) (width 0.2) (layer "B.Cu") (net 10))
 (segment (start 57.6 109.88) (end 58.35 109.13) (width 0.2) (layer "B.Cu") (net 10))
 (segment (start 59.3375 112.25) (end 58.78 112.25) (width 0.2) (layer "B.Cu") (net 10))
 (segment (start 62.89 109.13) (end 65.35 111.59) (width 0.2) (layer "B.Cu") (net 10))
 (segment (start 58.78 112.25) (end 57.6 111.07) (width 0.2) (layer "B.Cu") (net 10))
 (segment (start 65.35 111.59) (end 71.4432 111.59) (width 0.2) (layer "B.Cu") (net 10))
 (segment (start 57.6 111.07) (end 57.6 109.88) (width 0.2) (layer "B.Cu") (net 10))
 (segment (start 75.79 110.69) (end 75.79 109.55) (width 0.2) (layer "B.Cu") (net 11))
 (segment (start 75.79 109.55) (end 76.29 109.05) (width 0.2) (layer "B.Cu") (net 11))
 (segment (start 76.29 109.05) (end 77.59 109.05) (width 0.2) (layer "B.Cu") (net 11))
 (segment (start 78.907 110.9512) (end 76.0512 110.9512) (width 0.2) (layer "B.Cu") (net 11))
 (segment (start 85.27 119.9925) (end 85.27 117.3142) (width 0.2) (layer "B.Cu") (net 11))
 (segment (start 85.27 117.3142) (end 78.907 110.9512) (width 0.2) (layer "B.Cu") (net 11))
 (segment (start 76.0512 110.9512) (end 75.79 110.69) (width 0.2) (layer "B.Cu") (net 11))
 (segment (start 67.19 120.1925) (end 75.7925 111.59) (width 0.2) (layer "B.Cu") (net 2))
 (segment (start 75.7925 111.59) (end 77.59 111.59) (width 0.2) (layer "B.Cu") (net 2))
 (segment (start 75.94 106.9) (end 76.33 106.51) (width 0.2) (layer "B.Cu") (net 15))
 (segment (start 76.2188 108.4188) (end 75.94 108.14) (width 0.2) (layer "B.Cu") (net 15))
 (segment (start 76.33 106.51) (end 77.59 106.51) (width 0.2) (layer "B.Cu") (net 15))
 (segment (start 91.4763 108.4188) (end 76.2188 108.4188) (width 0.2) (layer "B.Cu") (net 15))
 (segment (start 75.94 108.14) (end 75.94 106.9) (width 0.2) (layer "B.Cu") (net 15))
 (segment (start 103.07 120.0125) (end 91.4763 108.4188) (width 0.2) (layer "B.Cu") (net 15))
 (segment (start 66.02 112.86) (end 71.4432 112.86) (width 0.2) (layer "B.Cu") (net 9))
 (segment (start 59.3375 110.25) (end 63.41 110.25) (width 0.2) (layer "B.Cu") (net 9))
 (segment (start 63.41 110.25) (end 66.02 112.86) (width 0.2) (layer "B.Cu") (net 9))
 (segment (start 101.2817 117.09) (end 91.5617 107.37) (width 0.2) (layer "B.Cu") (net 18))
 (segment (start 80.53 107.37) (end 79.0312 105.8712) (width 0.2) (layer "B.Cu") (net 18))
 (segment (start 120.53 119.9525) (end 117.6675 117.09) (width 0.2) (layer "B.Cu") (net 18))
 (segment (start 91.5617 107.37) (end 80.53 107.37) (width 0.2) (layer "B.Cu") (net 18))
 (segment (start 79.0312 105.8712) (end 76.4112 105.8712) (width 0.2) (layer "B.Cu") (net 18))
 (segment (start 76.38 103.97) (end 77.59 103.97) (width 0.2) (layer "B.Cu") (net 18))
 (segment (start 75.97 105.43) (end 75.97 104.38) (width 0.2) (layer "B.Cu") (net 18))
 (segment (start 117.6675 117.09) (end 101.2817 117.09) (width 0.2) (layer "B.Cu") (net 18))
 (segment (start 75.97 104.38) (end 76.38 103.97) (width 0.2) (layer "B.Cu") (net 18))
 (segment (start 76.4112 105.8712) (end 75.97 105.43) (width 0.2) (layer "B.Cu") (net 18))
 (segment (start 91.4046 107.78) (end 101.3346 117.71) (width 0.2) (layer "B.Cu") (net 16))
 (segment (start 102.7675 117.71) (end 105.07 120.0125) (width 0.2) (layer "B.Cu") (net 16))
 (segment (start 101.3346 117.71) (end 102.7675 117.71) (width 0.2) (layer "B.Cu") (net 16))
 (segment (start 77.59 107.78) (end 91.4046 107.78) (width 0.2) (layer "B.Cu") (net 16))
 (segment (start 87.27 118.73) (end 87.27 119.9925) (width 0.2) (layer "B.Cu") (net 12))
 (segment (start 78.86 110.32) (end 87.27 118.73) (width 0.2) (layer "B.Cu") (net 12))
 (segment (start 77.59 110.32) (end 78.86 110.32) (width 0.2) (layer "B.Cu") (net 12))
 (segment (start 100.34 112.75) (end 100.1 112.99) (width 0.5) (layer "F.Cu") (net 5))
 (segment (start 64.545 106.385) (end 64.545 105.43) (width 0.5) (layer "F.Cu") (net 5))
 (segment (start 65.21 111.49) (end 64.51 112.19) (width 0.5) (layer "F.Cu") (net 5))
 (segment (start 65.21 107.05) (end 66.33 105.93) (width 0.5) (layer "F.Cu") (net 5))
 (segment (start 100.635 112.665) (end 100.55 112.75) (width 0.5) (layer "F.Cu") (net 5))
 (segment (start 66.33 105.93) (end 66.33 105.26) (width 0.5) (layer "F.Cu") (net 5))
 (segment (start 64.51 112.19) (end 64.51 113.33) (width 0.5) (layer "F.Cu") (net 5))
 (segment (start 65.21 107.05) (end 64.545 106.385) (width 0.5) (layer "F.Cu") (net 5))
 (segment (start 82.62 112.99) (end 82.28 113.33) (width 0.5) (layer "F.Cu") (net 5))
 (segment (start 117.95 112.665) (end 100.635 112.665) (width 0.5) (layer "F.Cu") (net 5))
 (segment (start 100.1 112.99) (end 82.88 112.99) (width 0.5) (layer "F.Cu") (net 5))
 (segment (start 100.55 112.75) (end 100.34 112.75) (width 0.5) (layer "F.Cu") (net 5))
 (segment (start 64.715 105.26) (end 64.545 105.26) (width 0.5) (layer "F.Cu") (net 5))
 (segment (start 82.28 113.33) (end 64.51 113.33) (width 0.5) (layer "F.Cu") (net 5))
 (segment (start 65.21 110.29) (end 65.21 107.05) (width 0.5) (layer "F.Cu") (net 5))
 (segment (start 82.88 112.99) (end 82.62 112.99) (width 0.5) (layer "F.Cu") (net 5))
 (segment (start 65.21 110.29) (end 65.21 111.49) (width 0.5) (layer "F.Cu") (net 5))
 (segment (start 64.545 105.43) (end 64.715 105.26) (width 0.5) (layer "F.Cu") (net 5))
 (via (at 65.21 110.29) (size 0.6) (drill 0.3) (layers "F.Cu" "B.Cu") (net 5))
 (via (at 65.21 107.05) (size 0.6) (drill 0.3) (layers "F.Cu" "B.Cu") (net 5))
 (segment (start 65.21 110.29) (end 65.24 110.32) (width 0.5) (layer "B.Cu") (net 5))
 (segment (start 65.24 110.32) (end 71.4432 110.32) (width 0.5) (layer "B.Cu") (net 5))
 (segment (start 64.69 120.1925) (end 64.69 115.56) (width 0.2) (layer "F.Cu") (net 1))
 (segment (start 64.69 115.56) (end 64.51 115.38) (width 0.2) (layer "F.Cu") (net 1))
 (segment (start 82.88 115.04) (end 82.88 119.8825) (width 0.2) (layer "F.Cu") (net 6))
 (segment (start 82.88 119.8825) (end 82.77 119.9925) (width 0.2) (layer "F.Cu") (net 6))
 (segment (start 100.55 119.9925) (end 100.57 120.0125) (width 0.2) (layer "F.Cu") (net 14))
 (segment (start 100.55 114.8) (end 100.55 119.9925) (width 0.2) (layer "F.Cu") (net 14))
 (segment (start 117.95 114.715) (end 117.95 119.8725) (width 0.2) (layer "F.Cu") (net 17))
 (segment (start 117.95 119.8725) (end 118.03 119.9525) (width 0.2) (layer "F.Cu") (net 17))
 (segment (start 60.185 107.75) (end 62.495 105.44) (width 0.5) (layer "F.Cu") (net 8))
 (segment (start 62.495 105.44) (end 62.495 105.26) (width 0.5) (layer "F.Cu") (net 8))
 (segment (start 59.3375 107.75) (end 60.185 107.75) (width 0.5) (layer "F.Cu") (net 8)))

